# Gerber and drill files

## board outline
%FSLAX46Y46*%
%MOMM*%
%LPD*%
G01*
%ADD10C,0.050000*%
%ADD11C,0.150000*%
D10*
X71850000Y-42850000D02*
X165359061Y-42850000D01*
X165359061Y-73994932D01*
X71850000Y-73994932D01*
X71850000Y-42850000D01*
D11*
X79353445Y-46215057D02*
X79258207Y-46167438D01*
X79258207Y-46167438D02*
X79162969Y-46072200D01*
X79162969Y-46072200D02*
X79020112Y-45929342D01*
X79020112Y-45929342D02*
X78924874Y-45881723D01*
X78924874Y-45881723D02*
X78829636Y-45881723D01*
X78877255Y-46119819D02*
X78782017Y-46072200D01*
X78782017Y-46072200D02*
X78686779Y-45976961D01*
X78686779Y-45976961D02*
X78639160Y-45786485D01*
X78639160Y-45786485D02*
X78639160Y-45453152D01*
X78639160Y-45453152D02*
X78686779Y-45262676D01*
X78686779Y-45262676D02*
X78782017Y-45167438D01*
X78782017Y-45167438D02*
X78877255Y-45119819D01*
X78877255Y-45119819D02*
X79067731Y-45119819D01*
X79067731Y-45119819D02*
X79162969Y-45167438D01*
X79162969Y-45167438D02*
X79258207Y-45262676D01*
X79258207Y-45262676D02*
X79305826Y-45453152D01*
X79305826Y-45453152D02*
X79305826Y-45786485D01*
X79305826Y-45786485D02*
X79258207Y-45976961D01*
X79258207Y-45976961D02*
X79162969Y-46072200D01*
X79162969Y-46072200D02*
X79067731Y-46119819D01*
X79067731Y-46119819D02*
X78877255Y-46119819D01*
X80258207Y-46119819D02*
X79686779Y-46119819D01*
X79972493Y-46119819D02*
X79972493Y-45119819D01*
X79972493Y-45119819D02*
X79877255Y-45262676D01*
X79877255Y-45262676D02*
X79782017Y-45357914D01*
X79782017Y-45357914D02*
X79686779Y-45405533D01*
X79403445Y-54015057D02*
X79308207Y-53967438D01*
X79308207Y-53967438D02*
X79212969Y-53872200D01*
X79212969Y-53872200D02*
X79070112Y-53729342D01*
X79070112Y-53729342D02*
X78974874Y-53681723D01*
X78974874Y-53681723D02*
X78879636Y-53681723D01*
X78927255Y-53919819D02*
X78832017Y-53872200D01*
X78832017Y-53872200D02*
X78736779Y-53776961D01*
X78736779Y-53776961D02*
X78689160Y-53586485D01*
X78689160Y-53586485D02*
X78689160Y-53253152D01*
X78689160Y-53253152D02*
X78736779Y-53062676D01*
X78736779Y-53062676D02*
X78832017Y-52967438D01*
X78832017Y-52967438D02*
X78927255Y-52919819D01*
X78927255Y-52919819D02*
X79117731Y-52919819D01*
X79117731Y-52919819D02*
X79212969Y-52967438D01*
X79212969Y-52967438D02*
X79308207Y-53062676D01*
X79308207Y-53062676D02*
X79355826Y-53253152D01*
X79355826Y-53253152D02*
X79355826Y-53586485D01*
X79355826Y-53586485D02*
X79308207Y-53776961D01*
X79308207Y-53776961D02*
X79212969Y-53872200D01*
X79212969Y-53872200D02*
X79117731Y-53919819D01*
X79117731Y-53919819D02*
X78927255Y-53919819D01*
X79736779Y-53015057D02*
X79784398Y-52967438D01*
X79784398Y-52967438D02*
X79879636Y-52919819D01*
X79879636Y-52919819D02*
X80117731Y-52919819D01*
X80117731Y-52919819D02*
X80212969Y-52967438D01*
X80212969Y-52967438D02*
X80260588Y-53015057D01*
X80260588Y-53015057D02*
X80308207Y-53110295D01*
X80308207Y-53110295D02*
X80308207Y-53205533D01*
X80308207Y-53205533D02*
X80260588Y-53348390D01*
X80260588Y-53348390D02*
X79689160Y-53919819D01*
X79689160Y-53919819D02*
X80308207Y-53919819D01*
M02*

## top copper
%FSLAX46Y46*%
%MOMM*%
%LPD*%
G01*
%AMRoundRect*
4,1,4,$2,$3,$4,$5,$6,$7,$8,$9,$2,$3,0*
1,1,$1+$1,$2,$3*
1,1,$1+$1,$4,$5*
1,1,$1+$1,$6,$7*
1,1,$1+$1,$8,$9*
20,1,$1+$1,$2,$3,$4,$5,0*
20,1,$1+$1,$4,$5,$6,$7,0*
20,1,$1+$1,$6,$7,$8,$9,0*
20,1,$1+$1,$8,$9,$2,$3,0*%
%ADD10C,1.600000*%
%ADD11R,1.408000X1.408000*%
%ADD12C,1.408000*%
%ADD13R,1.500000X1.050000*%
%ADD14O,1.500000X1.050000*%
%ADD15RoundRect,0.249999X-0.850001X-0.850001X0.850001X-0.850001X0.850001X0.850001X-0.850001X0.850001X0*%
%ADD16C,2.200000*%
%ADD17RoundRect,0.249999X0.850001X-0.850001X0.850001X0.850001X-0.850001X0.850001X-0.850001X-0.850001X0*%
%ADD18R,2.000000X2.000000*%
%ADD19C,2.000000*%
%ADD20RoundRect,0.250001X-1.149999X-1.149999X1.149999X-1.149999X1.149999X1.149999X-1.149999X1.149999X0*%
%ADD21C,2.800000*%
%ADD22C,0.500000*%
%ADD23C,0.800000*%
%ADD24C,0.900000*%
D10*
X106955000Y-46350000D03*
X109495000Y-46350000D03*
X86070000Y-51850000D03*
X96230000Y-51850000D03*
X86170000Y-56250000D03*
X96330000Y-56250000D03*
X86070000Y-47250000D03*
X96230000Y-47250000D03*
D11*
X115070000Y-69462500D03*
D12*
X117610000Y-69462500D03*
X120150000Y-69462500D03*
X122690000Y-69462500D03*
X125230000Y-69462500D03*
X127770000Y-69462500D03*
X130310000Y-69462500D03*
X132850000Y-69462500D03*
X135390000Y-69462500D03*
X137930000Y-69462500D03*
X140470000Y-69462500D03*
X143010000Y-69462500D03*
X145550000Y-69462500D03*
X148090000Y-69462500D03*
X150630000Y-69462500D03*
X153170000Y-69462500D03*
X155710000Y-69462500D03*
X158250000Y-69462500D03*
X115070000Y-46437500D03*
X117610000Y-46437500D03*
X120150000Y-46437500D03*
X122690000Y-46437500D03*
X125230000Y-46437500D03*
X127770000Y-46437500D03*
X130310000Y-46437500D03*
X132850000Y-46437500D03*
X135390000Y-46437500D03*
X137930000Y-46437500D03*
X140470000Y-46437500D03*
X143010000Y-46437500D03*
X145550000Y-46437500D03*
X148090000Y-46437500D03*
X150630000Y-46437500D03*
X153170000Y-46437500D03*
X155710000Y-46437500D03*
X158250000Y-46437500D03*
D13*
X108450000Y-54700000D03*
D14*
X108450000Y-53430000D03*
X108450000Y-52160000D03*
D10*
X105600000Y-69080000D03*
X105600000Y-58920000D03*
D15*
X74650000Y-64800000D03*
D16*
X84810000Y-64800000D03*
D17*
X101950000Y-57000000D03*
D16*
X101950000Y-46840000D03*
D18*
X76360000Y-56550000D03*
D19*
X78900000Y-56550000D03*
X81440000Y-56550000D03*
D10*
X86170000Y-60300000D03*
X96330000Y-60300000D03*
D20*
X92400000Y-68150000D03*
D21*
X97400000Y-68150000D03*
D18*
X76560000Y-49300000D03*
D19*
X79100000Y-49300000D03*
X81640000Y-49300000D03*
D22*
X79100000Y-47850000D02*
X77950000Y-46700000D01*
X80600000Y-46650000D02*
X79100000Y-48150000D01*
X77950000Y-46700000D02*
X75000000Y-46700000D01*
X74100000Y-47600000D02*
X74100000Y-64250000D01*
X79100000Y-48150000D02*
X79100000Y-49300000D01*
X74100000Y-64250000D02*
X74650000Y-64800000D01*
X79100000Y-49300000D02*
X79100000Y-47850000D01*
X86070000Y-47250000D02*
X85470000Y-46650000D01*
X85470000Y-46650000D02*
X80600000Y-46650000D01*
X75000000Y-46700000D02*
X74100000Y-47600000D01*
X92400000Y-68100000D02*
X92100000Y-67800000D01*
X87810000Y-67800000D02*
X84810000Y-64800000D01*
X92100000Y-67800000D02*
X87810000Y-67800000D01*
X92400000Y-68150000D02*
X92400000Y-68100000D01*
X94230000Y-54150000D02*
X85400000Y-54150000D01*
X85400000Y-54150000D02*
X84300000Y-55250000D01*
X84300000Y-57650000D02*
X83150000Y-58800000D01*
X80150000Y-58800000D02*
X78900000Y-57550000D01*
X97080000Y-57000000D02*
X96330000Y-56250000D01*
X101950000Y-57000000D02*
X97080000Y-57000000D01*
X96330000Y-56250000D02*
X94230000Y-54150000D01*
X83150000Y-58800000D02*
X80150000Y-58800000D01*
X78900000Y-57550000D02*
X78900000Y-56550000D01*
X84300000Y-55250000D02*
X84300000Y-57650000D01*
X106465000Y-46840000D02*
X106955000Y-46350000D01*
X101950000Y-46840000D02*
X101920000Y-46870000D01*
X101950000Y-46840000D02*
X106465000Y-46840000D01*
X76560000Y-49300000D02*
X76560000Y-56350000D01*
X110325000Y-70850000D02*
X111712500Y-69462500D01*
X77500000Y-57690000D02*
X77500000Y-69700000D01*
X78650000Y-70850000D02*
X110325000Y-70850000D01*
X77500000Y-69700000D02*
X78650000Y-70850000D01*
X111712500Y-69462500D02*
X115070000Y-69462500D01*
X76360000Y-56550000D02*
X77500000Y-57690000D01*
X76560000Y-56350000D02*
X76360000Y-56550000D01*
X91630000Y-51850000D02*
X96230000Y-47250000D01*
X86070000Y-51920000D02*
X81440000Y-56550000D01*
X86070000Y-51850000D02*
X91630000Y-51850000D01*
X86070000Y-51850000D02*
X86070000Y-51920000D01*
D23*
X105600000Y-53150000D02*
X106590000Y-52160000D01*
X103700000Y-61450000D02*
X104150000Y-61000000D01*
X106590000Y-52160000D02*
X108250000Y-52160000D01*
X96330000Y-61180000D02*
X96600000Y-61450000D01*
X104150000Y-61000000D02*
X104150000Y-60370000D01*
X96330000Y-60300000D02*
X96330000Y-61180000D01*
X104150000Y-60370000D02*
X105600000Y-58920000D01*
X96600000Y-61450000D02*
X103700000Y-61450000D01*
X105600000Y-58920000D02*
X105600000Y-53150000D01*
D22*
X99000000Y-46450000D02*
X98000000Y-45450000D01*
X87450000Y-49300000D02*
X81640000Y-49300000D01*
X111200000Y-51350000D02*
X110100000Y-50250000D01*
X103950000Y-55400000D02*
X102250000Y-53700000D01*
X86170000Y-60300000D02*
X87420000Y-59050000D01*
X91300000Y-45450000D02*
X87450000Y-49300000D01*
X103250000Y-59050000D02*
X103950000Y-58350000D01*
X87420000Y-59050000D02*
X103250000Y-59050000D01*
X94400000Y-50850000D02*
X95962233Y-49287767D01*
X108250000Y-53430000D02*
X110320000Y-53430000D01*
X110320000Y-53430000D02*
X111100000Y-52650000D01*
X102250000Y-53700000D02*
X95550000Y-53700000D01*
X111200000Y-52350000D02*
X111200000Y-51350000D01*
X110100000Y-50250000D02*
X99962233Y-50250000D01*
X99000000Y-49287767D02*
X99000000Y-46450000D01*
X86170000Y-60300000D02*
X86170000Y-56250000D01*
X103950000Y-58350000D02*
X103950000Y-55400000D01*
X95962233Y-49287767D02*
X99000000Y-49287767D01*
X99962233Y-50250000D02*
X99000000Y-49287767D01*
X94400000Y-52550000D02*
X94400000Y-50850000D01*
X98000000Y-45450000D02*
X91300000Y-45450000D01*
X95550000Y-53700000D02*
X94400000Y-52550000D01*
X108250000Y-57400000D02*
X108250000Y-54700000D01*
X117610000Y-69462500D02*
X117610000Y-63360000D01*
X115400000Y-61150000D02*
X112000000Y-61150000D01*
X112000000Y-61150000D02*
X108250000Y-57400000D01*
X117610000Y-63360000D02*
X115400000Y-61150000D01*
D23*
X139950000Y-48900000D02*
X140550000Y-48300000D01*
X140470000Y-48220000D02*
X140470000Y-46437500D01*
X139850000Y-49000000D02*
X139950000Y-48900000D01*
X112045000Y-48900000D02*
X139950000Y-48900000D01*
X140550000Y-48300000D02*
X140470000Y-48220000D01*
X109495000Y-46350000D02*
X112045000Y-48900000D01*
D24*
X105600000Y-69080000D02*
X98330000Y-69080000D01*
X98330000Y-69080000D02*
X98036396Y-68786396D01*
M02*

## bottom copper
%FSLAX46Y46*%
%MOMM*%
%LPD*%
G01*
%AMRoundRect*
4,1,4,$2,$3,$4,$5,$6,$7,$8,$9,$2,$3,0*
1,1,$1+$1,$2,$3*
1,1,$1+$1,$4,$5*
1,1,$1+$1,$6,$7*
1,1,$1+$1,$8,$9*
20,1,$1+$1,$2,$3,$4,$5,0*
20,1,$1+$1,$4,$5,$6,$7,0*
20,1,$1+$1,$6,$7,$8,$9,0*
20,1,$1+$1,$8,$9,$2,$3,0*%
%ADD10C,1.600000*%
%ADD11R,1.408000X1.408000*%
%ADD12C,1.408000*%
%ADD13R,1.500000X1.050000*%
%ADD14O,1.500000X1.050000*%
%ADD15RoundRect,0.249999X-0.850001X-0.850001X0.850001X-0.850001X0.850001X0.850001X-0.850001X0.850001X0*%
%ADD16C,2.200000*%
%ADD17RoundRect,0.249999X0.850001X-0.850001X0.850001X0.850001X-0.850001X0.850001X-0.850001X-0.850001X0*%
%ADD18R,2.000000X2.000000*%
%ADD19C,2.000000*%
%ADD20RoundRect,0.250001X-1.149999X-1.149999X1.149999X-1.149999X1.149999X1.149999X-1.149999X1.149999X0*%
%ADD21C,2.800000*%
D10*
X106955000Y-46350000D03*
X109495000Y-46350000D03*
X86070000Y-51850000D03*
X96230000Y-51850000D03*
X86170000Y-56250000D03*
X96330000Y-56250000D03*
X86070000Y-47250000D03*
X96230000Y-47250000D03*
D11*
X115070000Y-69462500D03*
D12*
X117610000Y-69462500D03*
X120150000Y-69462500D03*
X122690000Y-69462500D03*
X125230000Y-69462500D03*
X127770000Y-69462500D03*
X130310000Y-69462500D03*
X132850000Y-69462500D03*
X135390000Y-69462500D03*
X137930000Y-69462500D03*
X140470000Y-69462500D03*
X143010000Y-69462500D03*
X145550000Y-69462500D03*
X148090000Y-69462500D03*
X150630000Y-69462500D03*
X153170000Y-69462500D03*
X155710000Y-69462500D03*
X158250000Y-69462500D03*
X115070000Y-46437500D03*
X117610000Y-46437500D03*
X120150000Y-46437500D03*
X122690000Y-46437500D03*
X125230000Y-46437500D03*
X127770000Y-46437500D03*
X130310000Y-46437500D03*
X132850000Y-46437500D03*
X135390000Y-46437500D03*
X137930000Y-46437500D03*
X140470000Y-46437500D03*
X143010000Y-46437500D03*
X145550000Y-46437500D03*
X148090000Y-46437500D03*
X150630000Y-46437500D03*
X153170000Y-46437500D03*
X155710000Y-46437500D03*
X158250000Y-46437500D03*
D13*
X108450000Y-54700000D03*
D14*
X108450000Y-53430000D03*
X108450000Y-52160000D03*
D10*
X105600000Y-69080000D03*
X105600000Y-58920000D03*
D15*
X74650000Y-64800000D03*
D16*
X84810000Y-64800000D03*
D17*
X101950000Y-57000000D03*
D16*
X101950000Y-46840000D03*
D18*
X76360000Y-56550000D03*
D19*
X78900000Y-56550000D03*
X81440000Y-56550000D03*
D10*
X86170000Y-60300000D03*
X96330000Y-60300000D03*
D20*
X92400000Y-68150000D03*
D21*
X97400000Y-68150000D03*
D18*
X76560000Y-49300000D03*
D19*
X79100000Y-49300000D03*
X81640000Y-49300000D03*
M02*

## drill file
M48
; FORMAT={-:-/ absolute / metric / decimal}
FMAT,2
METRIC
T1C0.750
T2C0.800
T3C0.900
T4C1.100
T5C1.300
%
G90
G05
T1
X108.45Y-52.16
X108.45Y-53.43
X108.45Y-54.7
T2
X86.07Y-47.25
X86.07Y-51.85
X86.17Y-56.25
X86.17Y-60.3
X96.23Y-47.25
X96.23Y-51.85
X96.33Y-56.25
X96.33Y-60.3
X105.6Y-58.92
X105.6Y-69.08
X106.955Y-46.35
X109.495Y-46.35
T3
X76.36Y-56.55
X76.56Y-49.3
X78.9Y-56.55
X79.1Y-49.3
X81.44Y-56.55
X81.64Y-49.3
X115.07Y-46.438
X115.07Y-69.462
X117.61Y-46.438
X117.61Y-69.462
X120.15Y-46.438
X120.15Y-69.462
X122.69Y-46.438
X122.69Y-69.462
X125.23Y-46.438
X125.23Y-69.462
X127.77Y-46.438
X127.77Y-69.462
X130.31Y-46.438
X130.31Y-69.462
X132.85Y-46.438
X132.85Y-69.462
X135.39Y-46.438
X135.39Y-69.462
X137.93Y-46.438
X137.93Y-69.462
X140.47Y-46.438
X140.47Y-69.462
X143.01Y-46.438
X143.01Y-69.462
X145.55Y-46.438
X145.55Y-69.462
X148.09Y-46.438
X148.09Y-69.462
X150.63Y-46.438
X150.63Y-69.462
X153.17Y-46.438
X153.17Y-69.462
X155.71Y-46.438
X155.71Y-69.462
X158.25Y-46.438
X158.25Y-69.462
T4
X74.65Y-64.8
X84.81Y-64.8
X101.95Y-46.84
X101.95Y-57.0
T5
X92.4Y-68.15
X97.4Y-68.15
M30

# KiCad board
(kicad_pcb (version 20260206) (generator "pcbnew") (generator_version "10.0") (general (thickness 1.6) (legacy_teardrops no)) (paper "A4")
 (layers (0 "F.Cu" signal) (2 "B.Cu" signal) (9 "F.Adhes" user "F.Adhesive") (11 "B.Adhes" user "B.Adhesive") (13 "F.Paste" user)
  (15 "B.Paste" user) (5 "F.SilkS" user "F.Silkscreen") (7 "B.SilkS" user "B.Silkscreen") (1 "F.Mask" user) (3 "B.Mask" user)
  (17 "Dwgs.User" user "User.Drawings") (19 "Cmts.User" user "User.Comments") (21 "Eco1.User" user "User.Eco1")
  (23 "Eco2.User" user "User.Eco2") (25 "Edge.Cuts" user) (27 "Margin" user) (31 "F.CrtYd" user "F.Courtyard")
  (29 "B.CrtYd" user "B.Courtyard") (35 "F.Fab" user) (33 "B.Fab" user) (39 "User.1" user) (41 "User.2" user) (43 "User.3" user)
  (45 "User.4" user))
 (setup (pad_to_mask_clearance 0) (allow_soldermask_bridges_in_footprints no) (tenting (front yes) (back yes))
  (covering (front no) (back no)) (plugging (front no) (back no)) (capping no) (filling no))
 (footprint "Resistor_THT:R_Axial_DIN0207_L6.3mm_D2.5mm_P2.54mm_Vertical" (layer "F.Cu") (at 106.955 46.35)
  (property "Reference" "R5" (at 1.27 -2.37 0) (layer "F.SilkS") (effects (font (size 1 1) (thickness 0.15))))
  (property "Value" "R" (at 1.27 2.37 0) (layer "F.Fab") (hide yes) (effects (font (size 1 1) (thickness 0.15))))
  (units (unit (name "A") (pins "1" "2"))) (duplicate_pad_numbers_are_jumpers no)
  (pad "1" thru_hole circle (at 0 0) (size 1.6 1.6) (drill 0.8) (layers "*.Cu" "*.Mask") (remove_unused_layers no) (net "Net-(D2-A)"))
  (pad "2" thru_hole circle (at 2.54 0) (size 1.6 1.6) (drill 0.8) (layers "*.Cu" "*.Mask") (remove_unused_layers no) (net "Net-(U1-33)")))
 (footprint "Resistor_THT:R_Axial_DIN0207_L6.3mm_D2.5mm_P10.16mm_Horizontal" (layer "F.Cu") (at 86.07 51.85)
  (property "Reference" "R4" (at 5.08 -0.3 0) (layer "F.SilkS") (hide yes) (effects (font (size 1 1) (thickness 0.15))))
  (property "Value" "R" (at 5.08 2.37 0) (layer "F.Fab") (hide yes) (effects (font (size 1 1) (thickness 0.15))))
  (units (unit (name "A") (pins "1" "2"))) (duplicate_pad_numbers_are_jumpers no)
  (pad "1" thru_hole circle (at 0 0) (size 1.6 1.6) (drill 0.8) (layers "*.Cu" "*.Mask") (remove_unused_layers no) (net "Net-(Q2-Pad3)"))
  (pad "2" thru_hole circle (at 10.16 0) (size 1.6 1.6) (drill 0.8) (layers "*.Cu" "*.Mask") (remove_unused_layers no) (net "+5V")))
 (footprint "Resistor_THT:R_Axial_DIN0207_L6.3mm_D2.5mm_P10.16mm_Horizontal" (layer "F.Cu") (at 86.17 56.25)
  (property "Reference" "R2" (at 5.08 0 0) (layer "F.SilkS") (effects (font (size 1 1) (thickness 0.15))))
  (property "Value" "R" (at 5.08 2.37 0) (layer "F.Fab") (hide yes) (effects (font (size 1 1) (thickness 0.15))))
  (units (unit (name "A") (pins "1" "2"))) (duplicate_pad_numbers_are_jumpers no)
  (pad "1" thru_hole circle (at 0 0) (size 1.6 1.6) (drill 0.8) (layers "*.Cu" "*.Mask") (remove_unused_layers no) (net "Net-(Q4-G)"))
  (pad "2" thru_hole circle (at 10.16 0) (size 1.6 1.6) (drill 0.8) (layers "*.Cu" "*.Mask") (remove_unused_layers no) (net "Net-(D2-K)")))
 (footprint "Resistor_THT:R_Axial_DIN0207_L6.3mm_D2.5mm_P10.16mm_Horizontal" (layer "F.Cu") (at 86.07 47.25)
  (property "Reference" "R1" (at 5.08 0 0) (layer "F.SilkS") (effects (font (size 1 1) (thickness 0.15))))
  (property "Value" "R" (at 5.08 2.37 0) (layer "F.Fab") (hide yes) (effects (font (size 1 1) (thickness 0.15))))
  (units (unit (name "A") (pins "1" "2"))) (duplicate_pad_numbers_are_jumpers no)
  (pad "1" thru_hole circle (at 0 0) (size 1.6 1.6) (drill 0.8) (layers "*.Cu" "*.Mask") (remove_unused_layers no) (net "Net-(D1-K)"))
  (pad "2" thru_hole circle (at 10.16 0) (size 1.6 1.6) (drill 0.8) (layers "*.Cu" "*.Mask") (remove_unused_layers no) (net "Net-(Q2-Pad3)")))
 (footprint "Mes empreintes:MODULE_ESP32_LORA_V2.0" (layer "F.Cu") (at 137.45 57.95)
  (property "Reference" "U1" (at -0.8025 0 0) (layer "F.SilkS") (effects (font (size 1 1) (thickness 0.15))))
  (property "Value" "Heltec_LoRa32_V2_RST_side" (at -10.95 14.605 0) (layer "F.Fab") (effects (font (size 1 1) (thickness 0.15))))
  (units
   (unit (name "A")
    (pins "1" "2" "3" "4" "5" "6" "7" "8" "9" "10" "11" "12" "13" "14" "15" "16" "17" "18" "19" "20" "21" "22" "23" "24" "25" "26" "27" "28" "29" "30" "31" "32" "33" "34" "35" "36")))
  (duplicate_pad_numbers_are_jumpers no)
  (pad "1" thru_hole rect (at -22.38 11.5125) (size 1.408 1.408) (drill 0.9) (layers "*.Cu" "*.Mask") (remove_unused_layers no) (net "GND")
   (solder_mask_margin 0.102))
  (pad "2" thru_hole circle (at -19.84 11.5125) (size 1.408 1.408) (drill 0.9) (layers "*.Cu" "*.Mask") (remove_unused_layers no)
   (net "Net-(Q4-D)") (solder_mask_margin 0.102))
  (pad "3" thru_hole circle (at -17.3 11.5125) (size 1.408 1.408) (drill 0.9) (layers "*.Cu" "*.Mask") (remove_unused_layers no)
   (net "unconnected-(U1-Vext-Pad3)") (solder_mask_margin 0.102))
  (pad "4" thru_hole circle (at -14.76 11.5125) (size 1.408 1.408) (drill 0.9) (layers "*.Cu" "*.Mask") (remove_unused_layers no)
   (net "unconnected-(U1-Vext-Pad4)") (solder_mask_margin 0.102))
  (pad "5" thru_hole circle (at -12.22 11.5125) (size 1.408 1.408) (drill 0.9) (layers "*.Cu" "*.Mask") (remove_unused_layers no)
   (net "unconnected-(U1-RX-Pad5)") (solder_mask_margin 0.102))
  (pad "6" thru_hole circle (at -9.68 11.5125) (size 1.408 1.408) (drill 0.9) (layers "*.Cu" "*.Mask") (remove_unused_layers no)
   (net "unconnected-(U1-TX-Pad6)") (solder_mask_margin 0.102))
  (pad "7" thru_hole circle (at -7.14 11.5125) (size 1.408 1.408) (drill 0.9) (layers "*.Cu" "*.Mask") (remove_unused_layers no)
   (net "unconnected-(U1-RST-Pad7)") (solder_mask_margin 0.102))
  (pad "8" thru_hole circle (at -4.6 11.5125) (size 1.408 1.408) (drill 0.9) (layers "*.Cu" "*.Mask") (remove_unused_layers no)
   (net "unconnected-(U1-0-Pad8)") (solder_mask_margin 0.102))
  (pad "9" thru_hole circle (at -2.06 11.5125) (size 1.408 1.408) (drill 0.9) (layers "*.Cu" "*.Mask") (remove_unused_layers no)
   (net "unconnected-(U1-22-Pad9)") (solder_mask_margin 0.102))
  (pad "10" thru_hole circle (at 0.48 11.5125) (size 1.408 1.408) (drill 0.9) (layers "*.Cu" "*.Mask") (remove_unused_layers no)
   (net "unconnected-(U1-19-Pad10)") (solder_mask_margin 0.102))
  (pad "11" thru_hole circle (at 3.02 11.5125) (size 1.408 1.408) (drill 0.9) (layers "*.Cu" "*.Mask") (remove_unused_layers no)
   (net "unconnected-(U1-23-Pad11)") (solder_mask_margin 0.102))
  (pad "12" thru_hole circle (at 5.56 11.5125) (size 1.408 1.408) (drill 0.9) (layers "*.Cu" "*.Mask") (remove_unused_layers no)
   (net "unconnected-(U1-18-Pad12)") (solder_mask_margin 0.102))
  (pad "13" thru_hole circle (at 8.1 11.5125) (size 1.408 1.408) (drill 0.9) (layers "*.Cu" "*.Mask") (remove_unused_layers no)
   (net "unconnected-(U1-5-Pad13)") (solder_mask_margin 0.102))
  (pad "14" thru_hole circle (at 10.64 11.5125) (size 1.408 1.408) (drill 0.9) (layers "*.Cu" "*.Mask") (remove_unused_layers no)
   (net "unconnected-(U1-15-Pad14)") (solder_mask_margin 0.102))
  (pad "15" thru_hole circle (at 13.18 11.5125) (size 1.408 1.408) (drill 0.9) (layers "*.Cu" "*.Mask") (remove_unused_layers no)
   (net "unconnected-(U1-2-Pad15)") (solder_mask_margin 0.102))
  (pad "16" thru_hole circle (at 15.72 11.5125) (size 1.408 1.408) (drill 0.9) (layers "*.Cu" "*.Mask") (remove_unused_layers no)
   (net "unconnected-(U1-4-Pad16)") (solder_mask_margin 0.102))
  (pad "17" thru_hole circle (at 18.26 11.5125) (size 1.408 1.408) (drill 0.9) (layers "*.Cu" "*.Mask") (remove_unused_layers no)
   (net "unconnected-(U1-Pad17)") (solder_mask_margin 0.102))
  (pad "18" thru_hole circle (at 20.8 11.5125) (size 1.408 1.408) (drill 0.9) (layers "*.Cu" "*.Mask") (remove_unused_layers no)
   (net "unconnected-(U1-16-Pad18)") (solder_mask_margin 0.102))
  (pad "19" thru_hole circle (at -22.38 -11.5125) (size 1.408 1.408) (drill 0.9) (layers "*.Cu" "*.Mask") (remove_unused_layers no)
   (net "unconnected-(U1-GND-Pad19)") (solder_mask_margin 0.102))
  (pad "20" thru_hole circle (at -19.84 -11.5125) (size 1.408 1.408) (drill 0.9) (layers "*.Cu" "*.Mask") (remove_unused_layers no)
   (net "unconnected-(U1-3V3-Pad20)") (solder_mask_margin 0.102))
  (pad "21" thru_hole circle (at -17.3 -11.5125) (size 1.408 1.408) (drill 0.9) (layers "*.Cu" "*.Mask") (remove_unused_layers no)
   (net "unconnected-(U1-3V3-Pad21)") (solder_mask_margin 0.102))
  (pad "22" thru_hole circle (at -14.76 -11.5125) (size 1.408 1.408) (drill 0.9) (layers "*.Cu" "*.Mask") (remove_unused_layers no)
   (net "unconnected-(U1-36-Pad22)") (solder_mask_margin 0.102))
  (pad "23" thru_hole circle (at -12.22 -11.5125) (size 1.408 1.408) (drill 0.9) (layers "*.Cu" "*.Mask") (remove_unused_layers no)
   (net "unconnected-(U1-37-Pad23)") (solder_mask_margin 0.102))
  (pad "24" thru_hole circle (at -9.68 -11.5125) (size 1.408 1.408) (drill 0.9) (layers "*.Cu" "*.Mask") (remove_unused_layers no)
   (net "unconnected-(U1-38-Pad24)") (solder_mask_margin 0.102))
  (pad "25" thru_hole circle (at -7.14 -11.5125) (size 1.408 1.408) (drill 0.9) (layers "*.Cu" "*.Mask") (remove_unused_layers no)
   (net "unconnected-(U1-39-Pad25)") (solder_mask_margin 0.102))
  (pad "26" thru_hole circle (at -4.6 -11.5125) (size 1.408 1.408) (drill 0.9) (layers "*.Cu" "*.Mask") (remove_unused_layers no)
   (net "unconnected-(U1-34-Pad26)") (solder_mask_margin 0.102))
  (pad "27" thru_hole circle (at -2.06 -11.5125) (size 1.408 1.408) (drill 0.9) (layers "*.Cu" "*.Mask") (remove_unused_layers no)
   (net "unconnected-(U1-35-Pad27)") (solder_mask_margin 0.102))
  (pad "28" thru_hole circle (at 0.48 -11.5125) (size 1.408 1.408) (drill 0.9) (layers "*.Cu" "*.Mask") (remove_unused_layers no)
   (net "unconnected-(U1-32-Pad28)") (solder_mask_margin 0.102))
  (pad "29" thru_hole circle (at 3.02 -11.5125) (size 1.408 1.408) (drill 0.9) (layers "*.Cu" "*.Mask") (remove_unused_layers no)
   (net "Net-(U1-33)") (solder_mask_margin 0.102))
  (pad "30" thru_hole circle (at 5.56 -11.5125) (size 1.408 1.408) (drill 0.9) (layers "*.Cu" "*.Mask") (remove_unused_layers no)
   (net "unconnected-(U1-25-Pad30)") (solder_mask_margin 0.102))
  (pad "31" thru_hole circle (at 8.1 -11.5125) (size 1.408 1.408) (drill 0.9) (layers "*.Cu" "*.Mask") (remove_unused_layers no)
   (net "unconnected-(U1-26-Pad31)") (solder_mask_margin 0.102))
  (pad "32" thru_hole circle (at 10.64 -11.5125) (size 1.408 1.408) (drill 0.9) (layers "*.Cu" "*.Mask") (remove_unused_layers no)
   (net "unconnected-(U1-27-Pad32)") (solder_mask_margin 0.102))
  (pad "33" thru_hole circle (at 13.18 -11.5125) (size 1.408 1.408) (drill 0.9) (layers "*.Cu" "*.Mask") (remove_unused_layers no)
   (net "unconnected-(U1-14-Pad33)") (solder_mask_margin 0.102))
  (pad "34" thru_hole circle (at 15.72 -11.5125) (size 1.408 1.408) (drill 0.9) (layers "*.Cu" "*.Mask") (remove_unused_layers no)
   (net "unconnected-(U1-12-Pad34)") (solder_mask_margin 0.102))
  (pad "35" thru_hole circle (at 18.26 -11.5125) (size 1.408 1.408) (drill 0.9) (layers "*.Cu" "*.Mask") (remove_unused_layers no)
   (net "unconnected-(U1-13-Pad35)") (solder_mask_margin 0.102))
  (pad "36" thru_hole circle (at 20.8 -11.5125) (size 1.408 1.408) (drill 0.9) (layers "*.Cu" "*.Mask") (remove_unused_layers no)
   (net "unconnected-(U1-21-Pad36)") (solder_mask_margin 0.102)))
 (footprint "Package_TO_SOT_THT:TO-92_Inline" (layer "F.Cu") (at 108.45 54.7 90)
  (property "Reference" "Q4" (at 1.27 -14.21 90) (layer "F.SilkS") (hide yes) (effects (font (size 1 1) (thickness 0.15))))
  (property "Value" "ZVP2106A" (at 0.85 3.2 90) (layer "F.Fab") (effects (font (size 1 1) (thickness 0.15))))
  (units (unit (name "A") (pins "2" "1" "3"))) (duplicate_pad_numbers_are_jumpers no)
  (pad "1" thru_hole rect (at 0 0 90) (size 1.05 1.5) (drill 0.75) (layers "*.Cu" "*.Mask") (remove_unused_layers no) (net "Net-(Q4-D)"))
  (pad "2" thru_hole oval (at 1.27 0 90) (size 1.05 1.5) (drill 0.75) (layers "*.Cu" "*.Mask") (remove_unused_layers no) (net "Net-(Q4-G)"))
  (pad "3" thru_hole oval (at 2.54 0 90) (size 1.05 1.5) (drill 0.75) (layers "*.Cu" "*.Mask") (remove_unused_layers no) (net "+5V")))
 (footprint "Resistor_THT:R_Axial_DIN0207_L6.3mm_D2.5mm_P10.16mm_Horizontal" (layer "F.Cu") (at 105.6 69.08 90)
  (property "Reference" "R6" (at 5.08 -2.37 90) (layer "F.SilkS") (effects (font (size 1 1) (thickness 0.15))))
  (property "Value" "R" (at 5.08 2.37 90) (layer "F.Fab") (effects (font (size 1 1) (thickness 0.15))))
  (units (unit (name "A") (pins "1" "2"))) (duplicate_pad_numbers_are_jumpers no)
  (pad "1" thru_hole circle (at 0 0 90) (size 1.6 1.6) (drill 0.8) (layers "*.Cu" "*.Mask") (remove_unused_layers no) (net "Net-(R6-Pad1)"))
  (pad "2" thru_hole circle (at 10.16 0 90) (size 1.6 1.6) (drill 0.8) (layers "*.Cu" "*.Mask") (remove_unused_layers no) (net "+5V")))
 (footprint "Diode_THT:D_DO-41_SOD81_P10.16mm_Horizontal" (layer "F.Cu") (at 74.65 64.8)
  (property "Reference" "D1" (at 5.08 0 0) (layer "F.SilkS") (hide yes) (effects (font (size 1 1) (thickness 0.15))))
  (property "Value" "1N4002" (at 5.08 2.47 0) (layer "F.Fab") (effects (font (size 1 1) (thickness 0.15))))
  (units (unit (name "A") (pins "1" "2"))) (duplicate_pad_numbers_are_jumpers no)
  (pad "1" thru_hole roundrect (at 0 0) (size 2.2 2.2) (drill 1.1) (layers "*.Cu" "*.Mask") (remove_unused_layers no)
   (roundrect_rratio 0.113636) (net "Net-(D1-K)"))
  (pad "2" thru_hole circle (at 10.16 0) (size 2.2 2.2) (drill 1.1) (layers "*.Cu" "*.Mask") (remove_unused_layers no) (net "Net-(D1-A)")))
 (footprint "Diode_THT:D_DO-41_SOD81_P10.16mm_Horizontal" (layer "F.Cu") (at 101.95 57 90)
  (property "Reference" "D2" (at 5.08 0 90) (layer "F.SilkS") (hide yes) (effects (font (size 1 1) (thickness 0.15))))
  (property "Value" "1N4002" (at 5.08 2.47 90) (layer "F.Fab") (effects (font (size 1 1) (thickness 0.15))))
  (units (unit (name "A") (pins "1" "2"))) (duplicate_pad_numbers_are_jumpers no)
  (pad "1" thru_hole roundrect (at 0 0 90) (size 2.2 2.2) (drill 1.1) (layers "*.Cu" "*.Mask") (remove_unused_layers no)
   (roundrect_rratio 0.113636) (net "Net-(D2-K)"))
  (pad "2" thru_hole circle (at 10.16 0 90) (size 2.2 2.2) (drill 1.1) (layers "*.Cu" "*.Mask") (remove_unused_layers no) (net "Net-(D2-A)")))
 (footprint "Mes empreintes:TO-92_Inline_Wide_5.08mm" (layer "F.Cu") (at 76.36 56.55)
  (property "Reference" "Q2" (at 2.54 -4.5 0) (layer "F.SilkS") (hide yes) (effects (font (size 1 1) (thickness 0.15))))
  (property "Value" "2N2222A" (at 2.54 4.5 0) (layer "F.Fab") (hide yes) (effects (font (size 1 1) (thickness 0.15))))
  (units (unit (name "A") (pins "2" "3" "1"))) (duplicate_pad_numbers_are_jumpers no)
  (pad "1" thru_hole rect (at 0 0) (size 2 2) (drill 0.9) (layers "*.Cu" "*.Mask") (remove_unused_layers no) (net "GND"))
  (pad "2" thru_hole circle (at 2.54 0) (size 2 2) (drill 0.9) (layers "*.Cu" "*.Mask") (remove_unused_layers no) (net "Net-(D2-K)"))
  (pad "3" thru_hole circle (at 5.08 0) (size 2 2) (drill 0.9) (layers "*.Cu" "*.Mask") (remove_unused_layers no) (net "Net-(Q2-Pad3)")))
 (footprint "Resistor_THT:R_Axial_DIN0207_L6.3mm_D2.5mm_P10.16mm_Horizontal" (layer "F.Cu") (at 86.17 60.3)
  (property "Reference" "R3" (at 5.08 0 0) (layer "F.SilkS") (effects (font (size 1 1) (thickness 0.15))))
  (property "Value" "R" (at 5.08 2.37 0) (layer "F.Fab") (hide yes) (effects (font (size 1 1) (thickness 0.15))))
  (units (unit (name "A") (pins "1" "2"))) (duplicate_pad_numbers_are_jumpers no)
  (pad "1" thru_hole circle (at 0 0) (size 1.6 1.6) (drill 0.8) (layers "*.Cu" "*.Mask") (remove_unused_layers no) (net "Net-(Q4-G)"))
  (pad "2" thru_hole circle (at 10.16 0) (size 1.6 1.6) (drill 0.8) (layers "*.Cu" "*.Mask") (remove_unused_layers no) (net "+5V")))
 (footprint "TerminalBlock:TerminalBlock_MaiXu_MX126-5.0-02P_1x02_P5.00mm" (layer "F.Cu") (at 92.4 68.15)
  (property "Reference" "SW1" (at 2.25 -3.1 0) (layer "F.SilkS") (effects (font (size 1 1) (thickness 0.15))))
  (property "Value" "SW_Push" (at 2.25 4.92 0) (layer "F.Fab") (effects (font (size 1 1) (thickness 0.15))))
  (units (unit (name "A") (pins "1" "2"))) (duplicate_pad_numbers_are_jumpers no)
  (pad "1" thru_hole roundrect (at 0 0) (size 2.8 2.8) (drill 1.3) (layers "*.Cu" "*.Mask") (remove_unused_layers no)
   (roundrect_rratio 0.089286) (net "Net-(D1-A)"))
  (pad "2" thru_hole circle (at 5 0) (size 2.8 2.8) (drill 1.3) (layers "*.Cu" "*.Mask") (remove_unused_layers no) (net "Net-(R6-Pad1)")))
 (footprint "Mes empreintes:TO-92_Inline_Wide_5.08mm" (layer "F.Cu") (at 76.56 49.3)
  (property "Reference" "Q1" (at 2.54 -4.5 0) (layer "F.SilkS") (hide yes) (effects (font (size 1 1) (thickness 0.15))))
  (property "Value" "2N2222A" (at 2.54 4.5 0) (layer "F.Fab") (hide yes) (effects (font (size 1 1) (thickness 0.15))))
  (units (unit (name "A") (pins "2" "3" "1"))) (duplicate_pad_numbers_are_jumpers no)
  (pad "1" thru_hole rect (at 0 0) (size 2 2) (drill 0.9) (layers "*.Cu" "*.Mask") (remove_unused_layers no) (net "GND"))
  (pad "2" thru_hole circle (at 2.54 0) (size 2 2) (drill 0.9) (layers "*.Cu" "*.Mask") (remove_unused_layers no) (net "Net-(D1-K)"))
  (pad "3" thru_hole circle (at 5.08 0) (size 2 2) (drill 0.9) (layers "*.Cu" "*.Mask") (remove_unused_layers no) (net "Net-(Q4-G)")))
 (gr_rect (start 71.85 42.85) (end 165.359061 73.994932) (stroke (width 0.05) (type default)) (fill no) (layer "Edge.Cuts"))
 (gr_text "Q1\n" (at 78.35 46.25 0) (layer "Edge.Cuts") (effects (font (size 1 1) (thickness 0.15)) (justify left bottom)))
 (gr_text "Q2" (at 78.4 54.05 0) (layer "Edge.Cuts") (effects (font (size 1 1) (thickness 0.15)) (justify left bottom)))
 (segment (start 79.1 47.85) (end 77.95 46.7) (width 0.5) (layer "F.Cu") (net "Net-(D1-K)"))
 (segment (start 80.6 46.65) (end 79.1 48.15) (width 0.5) (layer "F.Cu") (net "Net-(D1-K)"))
 (segment (start 77.95 46.7) (end 75 46.7) (width 0.5) (layer "F.Cu") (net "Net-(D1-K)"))
 (segment (start 74.1 47.6) (end 74.1 64.25) (width 0.5) (layer "F.Cu") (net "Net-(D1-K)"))
 (segment (start 79.1 48.15) (end 79.1 49.3) (width 0.5) (layer "F.Cu") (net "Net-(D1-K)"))
 (segment (start 74.1 64.25) (end 74.65 64.8) (width 0.5) (layer "F.Cu") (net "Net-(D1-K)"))
 (segment (start 79.1 49.3) (end 79.1 47.85) (width 0.5) (layer "F.Cu") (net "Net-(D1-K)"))
 (segment (start 86.07 47.25) (end 85.47 46.65) (width 0.5) (layer "F.Cu") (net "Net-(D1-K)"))
 (segment (start 85.47 46.65) (end 80.6 46.65) (width 0.5) (layer "F.Cu") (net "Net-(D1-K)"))
 (segment (start 75 46.7) (end 74.1 47.6) (width 0.5) (layer "F.Cu") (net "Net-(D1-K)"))
 (segment (start 92.4 68.1) (end 92.1 67.8) (width 0.5) (layer "F.Cu") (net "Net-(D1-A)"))
 (segment (start 87.81 67.8) (end 84.81 64.8) (width 0.5) (layer "F.Cu") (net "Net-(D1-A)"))
 (segment (start 92.1 67.8) (end 87.81 67.8) (width 0.5) (layer "F.Cu") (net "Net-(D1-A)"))
 (segment (start 92.4 68.15) (end 92.4 68.1) (width 0.5) (layer "F.Cu") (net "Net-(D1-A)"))
 (segment (start 94.23 54.15) (end 85.4 54.15) (width 0.5) (layer "F.Cu") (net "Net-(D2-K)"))
 (segment (start 85.4 54.15) (end 84.3 55.25) (width 0.5) (layer "F.Cu") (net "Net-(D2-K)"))
 (segment (start 84.3 57.65) (end 83.15 58.8) (width 0.5) (layer "F.Cu") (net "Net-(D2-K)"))
 (segment (start 80.15 58.8) (end 78.9 57.55) (width 0.5) (layer "F.Cu") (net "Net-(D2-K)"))
 (segment (start 97.08 57) (end 96.33 56.25) (width 0.5) (layer "F.Cu") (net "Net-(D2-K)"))
 (segment (start 101.95 57) (end 97.08 57) (width 0.5) (layer "F.Cu") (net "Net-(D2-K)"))
 (segment (start 96.33 56.25) (end 94.23 54.15) (width 0.5) (layer "F.Cu") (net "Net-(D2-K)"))
 (segment (start 83.15 58.8) (end 80.15 58.8) (width 0.5) (layer "F.Cu") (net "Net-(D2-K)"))
 (segment (start 78.9 57.55) (end 78.9 56.55) (width 0.5) (layer "F.Cu") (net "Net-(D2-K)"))
 (segment (start 84.3 55.25) (end 84.3 57.65) (width 0.5) (layer "F.Cu") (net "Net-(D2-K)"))
 (segment (start 106.465 46.84) (end 106.955 46.35) (width 0.5) (layer "F.Cu") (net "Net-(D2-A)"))
 (segment (start 101.95 46.84) (end 101.92 46.87) (width 0.5) (layer "F.Cu") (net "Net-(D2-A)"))
 (segment (start 101.95 46.84) (end 106.465 46.84) (width 0.5) (layer "F.Cu") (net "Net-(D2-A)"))
 (segment (start 76.56 49.3) (end 76.56 56.35) (width 0.5) (layer "F.Cu") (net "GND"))
 (segment (start 110.325 70.85) (end 111.7125 69.4625) (width 0.5) (layer "F.Cu") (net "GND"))
 (segment (start 77.5 57.69) (end 77.5 69.7) (width 0.5) (layer "F.Cu") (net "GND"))
 (segment (start 78.65 70.85) (end 110.325 70.85) (width 0.5) (layer "F.Cu") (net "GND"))
 (segment (start 77.5 69.7) (end 78.65 70.85) (width 0.5) (layer "F.Cu") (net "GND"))
 (segment (start 111.7125 69.4625) (end 115.07 69.4625) (width 0.5) (layer "F.Cu") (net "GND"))
 (segment (start 76.36 56.55) (end 77.5 57.69) (width 0.5) (layer "F.Cu") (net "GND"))
 (segment (start 76.56 56.35) (end 76.36 56.55) (width 0.5) (layer "F.Cu") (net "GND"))
 (segment (start 91.63 51.85) (end 96.23 47.25) (width 0.5) (layer "F.Cu") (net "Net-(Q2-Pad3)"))
 (segment (start 86.07 51.92) (end 81.44 56.55) (width 0.5) (layer "F.Cu") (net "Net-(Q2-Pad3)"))
 (segment (start 86.07 51.85) (end 91.63 51.85) (width 0.5) (layer "F.Cu") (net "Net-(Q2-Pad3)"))
 (segment (start 86.07 51.85) (end 86.07 51.92) (width 0.5) (layer "F.Cu") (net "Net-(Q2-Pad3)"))
 (segment (start 105.6 53.15) (end 106.59 52.16) (width 0.8) (layer "F.Cu") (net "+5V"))
 (segment (start 103.7 61.45) (end 104.15 61) (width 0.8) (layer "F.Cu") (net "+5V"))
 (segment (start 106.59 52.16) (end 108.25 52.16) (width 0.8) (layer "F.Cu") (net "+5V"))
 (segment (start 96.33 61.18) (end 96.6 61.45) (width 0.8) (layer "F.Cu") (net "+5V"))
 (segment (start 104.15 61) (end 104.15 60.37) (width 0.8) (layer "F.Cu") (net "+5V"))
 (segment (start 96.33 60.3) (end 96.33 61.18) (width 0.8) (layer "F.Cu") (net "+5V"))
 (segment (start 104.15 60.37) (end 105.6 58.92) (width 0.8) (layer "F.Cu") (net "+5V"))
 (segment (start 96.6 61.45) (end 103.7 61.45) (width 0.8) (layer "F.Cu") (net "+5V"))
 (segment (start 105.6 58.92) (end 105.6 53.15) (width 0.8) (layer "F.Cu") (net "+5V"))
 (segment (start 99 46.45) (end 98 45.45) (width 0.5) (layer "F.Cu") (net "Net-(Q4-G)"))
 (segment (start 87.45 49.3) (end 81.64 49.3) (width 0.5) (layer "F.Cu") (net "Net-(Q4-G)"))
 (segment (start 111.2 51.35) (end 110.1 50.25) (width 0.5) (layer "F.Cu") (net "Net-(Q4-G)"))
 (segment (start 103.95 55.4) (end 102.25 53.7) (width 0.5) (layer "F.Cu") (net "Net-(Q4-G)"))
 (segment (start 86.17 60.3) (end 87.42 59.05) (width 0.5) (layer "F.Cu") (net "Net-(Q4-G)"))
 (segment (start 91.3 45.45) (end 87.45 49.3) (width 0.5) (layer "F.Cu") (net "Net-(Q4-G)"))
 (segment (start 103.25 59.05) (end 103.95 58.35) (width 0.5) (layer "F.Cu") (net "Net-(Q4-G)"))
 (segment (start 87.42 59.05) (end 103.25 59.05) (width 0.5) (layer "F.Cu") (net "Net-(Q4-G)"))
 (segment (start 94.4 50.85) (end 95.962233 49.287767) (width 0.5) (layer "F.Cu") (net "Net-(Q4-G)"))
 (segment (start 108.25 53.43) (end 110.32 53.43) (width 0.5) (layer "F.Cu") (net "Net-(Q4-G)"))
 (segment (start 110.32 53.43) (end 111.1 52.65) (width 0.5) (layer "F.Cu") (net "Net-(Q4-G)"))
 (segment (start 102.25 53.7) (end 95.55 53.7) (width 0.5) (layer "F.Cu") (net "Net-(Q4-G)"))
 (segment (start 111.2 52.35) (end 111.2 51.35) (width 0.5) (layer "F.Cu") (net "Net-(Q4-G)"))
 (segment (start 110.1 50.25) (end 99.962233 50.25) (width 0.5) (layer "F.Cu") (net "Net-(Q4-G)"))
 (segment (start 99 49.287767) (end 99 46.45) (width 0.5) (layer "F.Cu") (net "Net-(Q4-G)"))
 (segment (start 86.17 60.3) (end 86.17 56.25) (width 0.5) (layer "F.Cu") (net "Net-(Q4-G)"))
 (segment (start 103.95 58.35) (end 103.95 55.4) (width 0.5) (layer "F.Cu") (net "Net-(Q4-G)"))
 (segment (start 95.962233 49.287767) (end 99 49.287767) (width 0.5) (layer "F.Cu") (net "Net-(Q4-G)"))
 (segment (start 99.962233 50.25) (end 99 49.287767) (width 0.5) (layer "F.Cu") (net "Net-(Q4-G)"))
 (segment (start 94.4 52.55) (end 94.4 50.85) (width 0.5) (layer "F.Cu") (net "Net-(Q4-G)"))
 (segment (start 98 45.45) (end 91.3 45.45) (width 0.5) (layer "F.Cu") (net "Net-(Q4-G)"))
 (segment (start 95.55 53.7) (end 94.4 52.55) (width 0.5) (layer "F.Cu") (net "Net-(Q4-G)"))
 (segment (start 108.25 57.4) (end 108.25 54.7) (width 0.5) (layer "F.Cu") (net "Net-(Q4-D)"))
 (segment (start 117.61 69.4625) (end 117.61 63.36) (width 0.5) (layer "F.Cu") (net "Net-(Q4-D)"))
 (segment (start 115.4 61.15) (end 112 61.15) (width 0.5) (layer "F.Cu") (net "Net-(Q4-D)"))
 (segment (start 112 61.15) (end 108.25 57.4) (width 0.5) (layer "F.Cu") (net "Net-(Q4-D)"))
 (segment (start 117.61 63.36) (end 115.4 61.15) (width 0.5) (layer "F.Cu") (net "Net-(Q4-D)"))
 (segment (start 139.95 48.9) (end 140.55 48.3) (width 0.8) (layer "F.Cu") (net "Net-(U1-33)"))
 (segment (start 140.47 48.22) (end 140.47 46.4375) (width 0.8) (layer "F.Cu") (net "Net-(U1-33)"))
 (segment (start 139.85 49) (end 139.95 48.9) (width 0.8) (layer "F.Cu") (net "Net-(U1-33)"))
 (segment (start 112.045 48.9) (end 139.95 48.9) (width 0.8) (layer "F.Cu") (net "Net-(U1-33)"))
 (segment (start 140.55 48.3) (end 140.47 48.22) (width 0.8) (layer "F.Cu") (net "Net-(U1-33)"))
 (segment (start 109.495 46.35) (end 112.045 48.9) (width 0.8) (layer "F.Cu") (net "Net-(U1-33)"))
 (segment (start 105.6 69.08) (end 98.33 69.08) (width 0.9) (layer "F.Cu") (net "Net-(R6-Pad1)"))
 (segment (start 98.33 69.08) (end 98.036396 68.786396) (width 0.9) (layer "F.Cu") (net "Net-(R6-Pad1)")))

